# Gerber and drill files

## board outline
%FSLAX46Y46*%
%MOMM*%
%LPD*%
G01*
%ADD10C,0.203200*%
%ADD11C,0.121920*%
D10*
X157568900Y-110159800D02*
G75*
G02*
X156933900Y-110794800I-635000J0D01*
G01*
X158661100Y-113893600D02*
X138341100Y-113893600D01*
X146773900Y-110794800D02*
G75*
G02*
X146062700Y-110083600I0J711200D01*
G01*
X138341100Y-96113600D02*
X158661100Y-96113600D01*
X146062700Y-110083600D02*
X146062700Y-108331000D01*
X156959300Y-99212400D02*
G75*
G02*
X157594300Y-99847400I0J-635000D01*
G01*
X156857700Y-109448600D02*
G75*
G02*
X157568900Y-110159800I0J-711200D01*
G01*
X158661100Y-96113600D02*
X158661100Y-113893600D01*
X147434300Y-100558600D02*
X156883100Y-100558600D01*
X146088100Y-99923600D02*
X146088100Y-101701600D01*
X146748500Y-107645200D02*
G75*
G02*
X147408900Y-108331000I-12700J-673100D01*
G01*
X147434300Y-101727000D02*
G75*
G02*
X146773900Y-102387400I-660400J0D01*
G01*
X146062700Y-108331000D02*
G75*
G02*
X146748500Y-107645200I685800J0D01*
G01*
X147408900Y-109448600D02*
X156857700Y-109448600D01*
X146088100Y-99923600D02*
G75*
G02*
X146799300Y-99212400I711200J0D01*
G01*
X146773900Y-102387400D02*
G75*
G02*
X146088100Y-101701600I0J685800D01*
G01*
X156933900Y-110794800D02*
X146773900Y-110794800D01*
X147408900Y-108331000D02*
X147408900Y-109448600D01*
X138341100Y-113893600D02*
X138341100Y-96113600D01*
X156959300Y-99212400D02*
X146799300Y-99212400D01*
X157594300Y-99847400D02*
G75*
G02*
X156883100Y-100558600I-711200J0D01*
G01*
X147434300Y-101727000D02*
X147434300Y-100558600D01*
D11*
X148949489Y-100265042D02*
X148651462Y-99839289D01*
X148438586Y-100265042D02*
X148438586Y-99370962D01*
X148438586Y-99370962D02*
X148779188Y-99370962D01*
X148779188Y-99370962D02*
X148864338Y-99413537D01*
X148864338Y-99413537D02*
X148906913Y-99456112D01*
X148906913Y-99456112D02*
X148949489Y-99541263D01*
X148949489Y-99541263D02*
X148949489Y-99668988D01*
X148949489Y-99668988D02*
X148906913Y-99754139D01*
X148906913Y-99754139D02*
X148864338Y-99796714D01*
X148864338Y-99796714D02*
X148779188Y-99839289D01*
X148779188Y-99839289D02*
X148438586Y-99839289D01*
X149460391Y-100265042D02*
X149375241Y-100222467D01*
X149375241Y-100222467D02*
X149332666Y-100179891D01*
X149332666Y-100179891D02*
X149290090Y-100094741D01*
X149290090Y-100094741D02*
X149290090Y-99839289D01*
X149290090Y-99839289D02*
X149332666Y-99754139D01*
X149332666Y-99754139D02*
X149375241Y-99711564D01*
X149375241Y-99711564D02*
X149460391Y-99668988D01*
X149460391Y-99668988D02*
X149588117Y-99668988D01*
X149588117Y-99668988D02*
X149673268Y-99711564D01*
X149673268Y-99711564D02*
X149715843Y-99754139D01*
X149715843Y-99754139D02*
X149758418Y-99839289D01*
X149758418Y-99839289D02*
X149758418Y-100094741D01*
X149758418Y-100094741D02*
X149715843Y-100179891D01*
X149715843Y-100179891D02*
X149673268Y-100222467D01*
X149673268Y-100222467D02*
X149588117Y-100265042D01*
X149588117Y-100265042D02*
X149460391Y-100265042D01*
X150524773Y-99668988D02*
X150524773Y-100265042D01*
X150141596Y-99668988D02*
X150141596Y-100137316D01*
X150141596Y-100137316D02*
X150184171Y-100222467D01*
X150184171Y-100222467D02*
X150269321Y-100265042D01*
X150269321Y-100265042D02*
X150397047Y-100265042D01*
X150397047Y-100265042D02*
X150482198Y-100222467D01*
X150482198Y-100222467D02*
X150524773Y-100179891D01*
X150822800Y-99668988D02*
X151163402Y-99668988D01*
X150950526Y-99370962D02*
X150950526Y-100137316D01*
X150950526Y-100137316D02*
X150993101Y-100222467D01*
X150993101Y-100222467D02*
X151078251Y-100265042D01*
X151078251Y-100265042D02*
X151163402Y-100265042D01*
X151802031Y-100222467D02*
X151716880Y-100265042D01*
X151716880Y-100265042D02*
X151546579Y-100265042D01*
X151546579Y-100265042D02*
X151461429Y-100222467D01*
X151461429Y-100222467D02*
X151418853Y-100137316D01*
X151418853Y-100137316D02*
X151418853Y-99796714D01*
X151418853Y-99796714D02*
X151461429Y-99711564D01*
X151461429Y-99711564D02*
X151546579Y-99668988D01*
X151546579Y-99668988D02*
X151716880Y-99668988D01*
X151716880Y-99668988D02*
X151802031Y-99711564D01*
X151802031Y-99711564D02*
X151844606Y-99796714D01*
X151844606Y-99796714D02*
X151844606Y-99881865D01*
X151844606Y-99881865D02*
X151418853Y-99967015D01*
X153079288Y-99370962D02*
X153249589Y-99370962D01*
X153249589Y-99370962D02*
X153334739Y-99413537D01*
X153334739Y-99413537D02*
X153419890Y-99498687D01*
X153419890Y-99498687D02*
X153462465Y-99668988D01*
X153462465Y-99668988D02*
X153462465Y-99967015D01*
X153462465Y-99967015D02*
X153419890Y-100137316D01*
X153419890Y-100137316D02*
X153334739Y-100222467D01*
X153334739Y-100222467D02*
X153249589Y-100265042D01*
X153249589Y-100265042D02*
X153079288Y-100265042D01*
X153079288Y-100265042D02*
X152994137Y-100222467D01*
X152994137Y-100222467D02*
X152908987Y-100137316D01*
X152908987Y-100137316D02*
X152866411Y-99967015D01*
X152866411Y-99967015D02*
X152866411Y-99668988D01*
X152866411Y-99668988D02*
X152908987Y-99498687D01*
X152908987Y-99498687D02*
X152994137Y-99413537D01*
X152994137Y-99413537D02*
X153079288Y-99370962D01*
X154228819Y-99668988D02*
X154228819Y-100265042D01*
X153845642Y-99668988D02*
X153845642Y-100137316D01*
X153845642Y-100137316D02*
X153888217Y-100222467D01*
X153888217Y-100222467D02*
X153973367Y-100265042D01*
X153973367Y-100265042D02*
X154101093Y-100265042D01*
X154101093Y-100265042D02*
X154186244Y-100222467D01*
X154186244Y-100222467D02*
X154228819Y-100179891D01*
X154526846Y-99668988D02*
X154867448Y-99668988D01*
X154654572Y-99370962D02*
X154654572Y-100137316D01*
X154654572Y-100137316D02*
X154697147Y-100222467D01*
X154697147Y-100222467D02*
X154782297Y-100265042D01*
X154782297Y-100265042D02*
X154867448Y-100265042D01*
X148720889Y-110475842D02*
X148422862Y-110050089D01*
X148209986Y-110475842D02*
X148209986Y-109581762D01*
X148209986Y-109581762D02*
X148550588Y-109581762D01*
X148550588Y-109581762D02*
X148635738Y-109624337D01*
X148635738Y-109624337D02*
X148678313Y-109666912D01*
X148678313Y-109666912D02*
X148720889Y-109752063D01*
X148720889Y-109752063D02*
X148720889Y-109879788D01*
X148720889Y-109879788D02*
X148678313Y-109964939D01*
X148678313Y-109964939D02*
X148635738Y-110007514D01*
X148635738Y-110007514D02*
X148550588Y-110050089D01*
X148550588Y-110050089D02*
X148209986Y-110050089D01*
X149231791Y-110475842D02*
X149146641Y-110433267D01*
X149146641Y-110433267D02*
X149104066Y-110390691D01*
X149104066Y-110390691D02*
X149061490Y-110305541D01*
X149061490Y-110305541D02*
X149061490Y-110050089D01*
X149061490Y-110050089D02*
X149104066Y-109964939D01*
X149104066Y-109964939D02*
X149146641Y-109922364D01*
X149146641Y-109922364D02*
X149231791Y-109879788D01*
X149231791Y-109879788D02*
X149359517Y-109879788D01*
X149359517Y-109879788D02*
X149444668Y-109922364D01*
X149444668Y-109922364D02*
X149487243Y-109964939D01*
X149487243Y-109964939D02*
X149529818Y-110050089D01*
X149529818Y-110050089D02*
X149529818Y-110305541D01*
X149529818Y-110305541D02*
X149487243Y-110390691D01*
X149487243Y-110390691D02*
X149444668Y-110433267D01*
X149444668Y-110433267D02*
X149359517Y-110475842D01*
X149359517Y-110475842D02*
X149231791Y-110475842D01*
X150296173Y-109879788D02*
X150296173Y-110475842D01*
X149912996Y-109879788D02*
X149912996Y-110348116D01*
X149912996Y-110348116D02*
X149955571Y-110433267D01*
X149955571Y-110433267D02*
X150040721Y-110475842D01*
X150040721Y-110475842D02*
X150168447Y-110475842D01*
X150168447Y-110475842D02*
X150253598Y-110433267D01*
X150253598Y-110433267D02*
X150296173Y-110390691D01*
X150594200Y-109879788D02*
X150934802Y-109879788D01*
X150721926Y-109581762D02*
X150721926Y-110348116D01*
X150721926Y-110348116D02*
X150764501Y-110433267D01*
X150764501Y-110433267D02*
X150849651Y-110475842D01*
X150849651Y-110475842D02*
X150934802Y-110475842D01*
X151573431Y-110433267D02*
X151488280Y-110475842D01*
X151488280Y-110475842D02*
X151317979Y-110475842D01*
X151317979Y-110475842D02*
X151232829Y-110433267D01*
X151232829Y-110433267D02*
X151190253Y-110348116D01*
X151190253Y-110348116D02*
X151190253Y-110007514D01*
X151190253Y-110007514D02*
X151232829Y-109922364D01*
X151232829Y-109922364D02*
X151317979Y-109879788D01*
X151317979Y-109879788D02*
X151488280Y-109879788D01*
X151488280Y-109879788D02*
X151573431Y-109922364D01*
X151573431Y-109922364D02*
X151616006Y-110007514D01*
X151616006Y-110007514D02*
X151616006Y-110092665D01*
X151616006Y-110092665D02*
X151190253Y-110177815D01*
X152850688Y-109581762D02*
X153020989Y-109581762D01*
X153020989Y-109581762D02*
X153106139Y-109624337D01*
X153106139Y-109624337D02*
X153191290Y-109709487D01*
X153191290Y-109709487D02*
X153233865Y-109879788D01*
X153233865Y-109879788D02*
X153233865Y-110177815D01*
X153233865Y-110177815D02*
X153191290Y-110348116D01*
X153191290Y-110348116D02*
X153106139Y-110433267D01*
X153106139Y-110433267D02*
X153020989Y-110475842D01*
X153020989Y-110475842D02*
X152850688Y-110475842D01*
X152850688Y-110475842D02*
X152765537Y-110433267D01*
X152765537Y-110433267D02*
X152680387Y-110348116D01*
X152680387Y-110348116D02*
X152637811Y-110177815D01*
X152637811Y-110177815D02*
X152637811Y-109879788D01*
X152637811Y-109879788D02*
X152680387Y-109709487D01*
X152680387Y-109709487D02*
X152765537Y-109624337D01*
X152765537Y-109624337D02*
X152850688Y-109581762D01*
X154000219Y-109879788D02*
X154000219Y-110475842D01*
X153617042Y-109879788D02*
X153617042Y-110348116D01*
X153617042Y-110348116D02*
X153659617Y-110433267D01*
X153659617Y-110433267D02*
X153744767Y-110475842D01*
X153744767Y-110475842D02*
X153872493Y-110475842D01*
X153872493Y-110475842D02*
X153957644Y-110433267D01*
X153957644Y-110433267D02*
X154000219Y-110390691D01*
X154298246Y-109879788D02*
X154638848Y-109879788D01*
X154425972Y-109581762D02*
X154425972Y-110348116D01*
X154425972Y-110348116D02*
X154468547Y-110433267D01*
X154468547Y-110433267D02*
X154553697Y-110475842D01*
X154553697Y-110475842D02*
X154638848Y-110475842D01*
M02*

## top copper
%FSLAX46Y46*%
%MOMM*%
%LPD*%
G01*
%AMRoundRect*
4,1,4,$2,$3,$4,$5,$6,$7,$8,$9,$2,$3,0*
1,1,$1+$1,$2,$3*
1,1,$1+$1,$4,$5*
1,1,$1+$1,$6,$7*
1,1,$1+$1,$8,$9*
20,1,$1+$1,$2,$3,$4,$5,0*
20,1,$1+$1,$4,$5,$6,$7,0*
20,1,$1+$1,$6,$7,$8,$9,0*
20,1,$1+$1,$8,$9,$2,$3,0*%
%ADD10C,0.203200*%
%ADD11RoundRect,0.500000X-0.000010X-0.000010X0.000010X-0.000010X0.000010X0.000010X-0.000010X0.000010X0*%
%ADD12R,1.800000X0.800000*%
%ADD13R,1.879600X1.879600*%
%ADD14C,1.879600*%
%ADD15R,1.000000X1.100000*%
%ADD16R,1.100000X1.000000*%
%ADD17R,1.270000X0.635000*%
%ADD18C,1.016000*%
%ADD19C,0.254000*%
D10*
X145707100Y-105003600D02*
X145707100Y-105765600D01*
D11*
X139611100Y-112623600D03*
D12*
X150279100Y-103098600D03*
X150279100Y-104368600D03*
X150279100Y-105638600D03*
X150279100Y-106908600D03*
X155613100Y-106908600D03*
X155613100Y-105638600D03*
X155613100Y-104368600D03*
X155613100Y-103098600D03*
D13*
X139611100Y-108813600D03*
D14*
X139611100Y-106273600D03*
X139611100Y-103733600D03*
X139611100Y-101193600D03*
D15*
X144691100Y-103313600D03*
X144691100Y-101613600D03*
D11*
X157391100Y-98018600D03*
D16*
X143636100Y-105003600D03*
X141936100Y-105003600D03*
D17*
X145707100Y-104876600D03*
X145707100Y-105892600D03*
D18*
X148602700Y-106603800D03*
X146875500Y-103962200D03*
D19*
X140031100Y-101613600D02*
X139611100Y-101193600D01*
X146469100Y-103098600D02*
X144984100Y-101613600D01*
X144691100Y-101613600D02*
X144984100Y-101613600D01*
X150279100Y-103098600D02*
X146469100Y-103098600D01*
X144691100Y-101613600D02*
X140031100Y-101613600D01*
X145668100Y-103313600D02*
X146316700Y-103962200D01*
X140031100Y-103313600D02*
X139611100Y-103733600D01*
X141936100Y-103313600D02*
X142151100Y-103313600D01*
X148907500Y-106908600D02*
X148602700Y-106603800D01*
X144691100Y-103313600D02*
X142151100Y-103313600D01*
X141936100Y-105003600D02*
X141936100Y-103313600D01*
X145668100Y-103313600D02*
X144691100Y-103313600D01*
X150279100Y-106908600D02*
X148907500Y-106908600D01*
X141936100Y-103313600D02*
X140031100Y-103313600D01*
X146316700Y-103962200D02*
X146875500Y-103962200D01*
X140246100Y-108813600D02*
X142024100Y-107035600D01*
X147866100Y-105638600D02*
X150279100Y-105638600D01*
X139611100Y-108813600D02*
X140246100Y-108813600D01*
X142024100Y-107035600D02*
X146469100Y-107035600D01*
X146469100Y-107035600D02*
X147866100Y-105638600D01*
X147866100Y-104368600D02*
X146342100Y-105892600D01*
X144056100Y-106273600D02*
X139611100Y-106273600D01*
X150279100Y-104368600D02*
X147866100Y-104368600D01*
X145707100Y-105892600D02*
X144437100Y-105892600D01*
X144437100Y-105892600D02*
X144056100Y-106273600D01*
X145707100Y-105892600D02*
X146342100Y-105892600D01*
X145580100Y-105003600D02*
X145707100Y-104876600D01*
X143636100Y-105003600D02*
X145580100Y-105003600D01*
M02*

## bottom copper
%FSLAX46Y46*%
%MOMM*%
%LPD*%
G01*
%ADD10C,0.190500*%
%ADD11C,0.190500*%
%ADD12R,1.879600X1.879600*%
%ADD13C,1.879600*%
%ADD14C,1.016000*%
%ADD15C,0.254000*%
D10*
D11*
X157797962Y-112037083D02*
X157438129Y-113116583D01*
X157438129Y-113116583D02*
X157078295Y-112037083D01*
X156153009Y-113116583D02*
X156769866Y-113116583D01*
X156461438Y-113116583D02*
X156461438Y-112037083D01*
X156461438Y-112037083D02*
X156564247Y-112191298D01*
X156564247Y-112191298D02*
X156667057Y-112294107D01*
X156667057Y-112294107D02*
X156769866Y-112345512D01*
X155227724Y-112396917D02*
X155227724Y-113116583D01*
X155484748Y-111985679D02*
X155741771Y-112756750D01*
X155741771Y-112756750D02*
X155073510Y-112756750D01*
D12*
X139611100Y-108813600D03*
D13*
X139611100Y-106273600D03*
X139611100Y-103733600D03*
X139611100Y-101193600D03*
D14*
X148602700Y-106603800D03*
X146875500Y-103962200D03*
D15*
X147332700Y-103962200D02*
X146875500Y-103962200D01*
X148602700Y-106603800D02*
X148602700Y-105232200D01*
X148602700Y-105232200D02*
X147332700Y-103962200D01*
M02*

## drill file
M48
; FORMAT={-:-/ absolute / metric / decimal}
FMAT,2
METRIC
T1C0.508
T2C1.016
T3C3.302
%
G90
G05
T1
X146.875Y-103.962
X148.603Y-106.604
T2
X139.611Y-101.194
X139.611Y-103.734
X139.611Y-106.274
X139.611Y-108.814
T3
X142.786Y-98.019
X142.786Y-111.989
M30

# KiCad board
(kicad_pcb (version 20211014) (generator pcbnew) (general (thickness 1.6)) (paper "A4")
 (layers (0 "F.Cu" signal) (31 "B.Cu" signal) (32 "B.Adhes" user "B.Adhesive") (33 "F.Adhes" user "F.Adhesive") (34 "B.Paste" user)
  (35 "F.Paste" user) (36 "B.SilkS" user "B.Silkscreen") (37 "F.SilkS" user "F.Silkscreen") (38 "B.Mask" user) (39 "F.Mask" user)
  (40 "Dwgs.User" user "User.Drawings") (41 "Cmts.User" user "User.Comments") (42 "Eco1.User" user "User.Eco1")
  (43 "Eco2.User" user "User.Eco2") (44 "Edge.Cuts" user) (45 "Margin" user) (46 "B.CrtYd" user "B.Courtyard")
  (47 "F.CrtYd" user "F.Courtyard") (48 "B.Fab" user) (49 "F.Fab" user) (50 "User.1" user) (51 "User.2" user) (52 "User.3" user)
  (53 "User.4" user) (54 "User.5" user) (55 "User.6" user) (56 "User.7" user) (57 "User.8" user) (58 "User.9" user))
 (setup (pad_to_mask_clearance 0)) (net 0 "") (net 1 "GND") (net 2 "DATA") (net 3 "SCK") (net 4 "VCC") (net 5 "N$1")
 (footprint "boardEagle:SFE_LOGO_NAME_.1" (layer "F.Cu") (at 145.2245 99.568)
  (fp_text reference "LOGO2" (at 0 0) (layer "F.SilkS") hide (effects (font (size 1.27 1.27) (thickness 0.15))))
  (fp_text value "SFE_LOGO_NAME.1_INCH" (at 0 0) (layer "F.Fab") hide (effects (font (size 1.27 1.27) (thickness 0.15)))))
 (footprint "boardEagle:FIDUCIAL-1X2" (layer "F.Cu") (at 139.6111 112.6236)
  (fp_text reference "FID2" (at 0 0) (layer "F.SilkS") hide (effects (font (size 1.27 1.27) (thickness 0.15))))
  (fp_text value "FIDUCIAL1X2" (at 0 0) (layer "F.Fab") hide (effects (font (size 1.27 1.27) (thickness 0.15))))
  (pad "1" smd roundrect (at 0 0) (size 1 1) (layers "F.Cu" "F.Mask") (roundrect_rratio 0.5) (solder_mask_margin 0.1016)))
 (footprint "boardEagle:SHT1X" (layer "F.Cu") (at 152.9461 105.0036)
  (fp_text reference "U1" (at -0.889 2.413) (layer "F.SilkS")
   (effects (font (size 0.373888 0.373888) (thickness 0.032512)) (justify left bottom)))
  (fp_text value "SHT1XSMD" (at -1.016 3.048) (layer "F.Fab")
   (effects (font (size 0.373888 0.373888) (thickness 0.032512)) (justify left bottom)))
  (pad "1" smd rect (at -2.667 -1.905 180) (size 1.8 0.8) (layers "F.Cu" "F.Paste" "F.Mask") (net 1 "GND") (solder_mask_margin 0.1016))
  (pad "2" smd rect (at -2.667 -0.635 180) (size 1.8 0.8) (layers "F.Cu" "F.Paste" "F.Mask") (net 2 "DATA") (solder_mask_margin 0.1016))
  (pad "3" smd rect (at -2.667 0.635 180) (size 1.8 0.8) (layers "F.Cu" "F.Paste" "F.Mask") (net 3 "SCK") (solder_mask_margin 0.1016))
  (pad "4" smd rect (at -2.667 1.905 180) (size 1.8 0.8) (layers "F.Cu" "F.Paste" "F.Mask") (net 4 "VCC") (solder_mask_margin 0.1016))
  (pad "5" smd rect (at 2.667 1.905 180) (size 1.8 0.8) (layers "F.Cu" "F.Paste" "F.Mask") (solder_mask_margin 0.1016))
  (pad "6" smd rect (at 2.667 0.635 180) (size 1.8 0.8) (layers "F.Cu" "F.Paste" "F.Mask") (solder_mask_margin 0.1016))
  (pad "7" smd rect (at 2.667 -0.635 180) (size 1.8 0.8) (layers "F.Cu" "F.Paste" "F.Mask") (solder_mask_margin 0.1016))
  (pad "8" smd rect (at 2.667 -1.905 180) (size 1.8 0.8) (layers "F.Cu" "F.Paste" "F.Mask") (solder_mask_margin 0.1016)))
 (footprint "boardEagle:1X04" (layer "F.Cu") (at 139.6111 108.8136 90)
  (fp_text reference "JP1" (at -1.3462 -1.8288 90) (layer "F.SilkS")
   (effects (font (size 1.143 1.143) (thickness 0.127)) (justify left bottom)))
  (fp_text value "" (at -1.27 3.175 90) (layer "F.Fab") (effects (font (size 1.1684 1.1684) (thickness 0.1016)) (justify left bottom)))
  (pad "1" thru_hole rect (at 0 0 180) (size 1.8796 1.8796) (drill 1.016) (layers *.Cu *.Mask) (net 3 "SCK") (solder_mask_margin 0.1016))
  (pad "2" thru_hole circle (at 2.54 0 180) (size 1.8796 1.8796) (drill 1.016) (layers *.Cu *.Mask) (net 2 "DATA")
   (solder_mask_margin 0.1016))
  (pad "3" thru_hole circle (at 5.08 0 180) (size 1.8796 1.8796) (drill 1.016) (layers *.Cu *.Mask) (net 4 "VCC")
   (solder_mask_margin 0.1016))
  (pad "4" thru_hole circle (at 7.62 0 180) (size 1.8796 1.8796) (drill 1.016) (layers *.Cu *.Mask) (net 1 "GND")
   (solder_mask_margin 0.1016)))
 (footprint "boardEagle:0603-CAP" (layer "F.Cu") (at 144.6911 102.4636 90)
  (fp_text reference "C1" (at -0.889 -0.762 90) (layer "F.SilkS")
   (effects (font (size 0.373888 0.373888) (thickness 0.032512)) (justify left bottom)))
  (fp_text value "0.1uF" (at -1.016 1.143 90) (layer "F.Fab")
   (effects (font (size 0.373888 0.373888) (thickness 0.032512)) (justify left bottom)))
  (pad "1" smd rect (at -0.85 0 90) (size 1.1 1) (layers "F.Cu" "F.Paste" "F.Mask") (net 4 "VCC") (solder_mask_margin 0.1016))
  (pad "2" smd rect (at 0.85 0 90) (size 1.1 1) (layers "F.Cu" "F.Paste" "F.Mask") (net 1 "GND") (solder_mask_margin 0.1016)))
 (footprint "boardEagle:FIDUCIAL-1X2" (layer "F.Cu") (at 157.3911 98.0186)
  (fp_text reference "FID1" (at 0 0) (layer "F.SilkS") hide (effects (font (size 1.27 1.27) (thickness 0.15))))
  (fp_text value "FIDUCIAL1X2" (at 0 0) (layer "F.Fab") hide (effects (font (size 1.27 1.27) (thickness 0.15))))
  (pad "1" smd roundrect (at 0 0) (size 1 1) (layers "F.Cu" "F.Mask") (roundrect_rratio 0.5) (solder_mask_margin 0.1016)))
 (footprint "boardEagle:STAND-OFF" (layer "F.Cu") (at 142.7861 111.9886)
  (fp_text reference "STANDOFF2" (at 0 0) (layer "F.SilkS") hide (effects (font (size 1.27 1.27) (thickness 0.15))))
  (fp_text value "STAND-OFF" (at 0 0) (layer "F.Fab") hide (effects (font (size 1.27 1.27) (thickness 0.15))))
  (pad "" np_thru_hole circle (at 0 0) (size 3.302 3.302) (drill 3.302) (layers *.Cu *.Mask)))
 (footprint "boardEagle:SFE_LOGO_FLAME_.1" (layer "F.Cu") (at 138.5189 99.695)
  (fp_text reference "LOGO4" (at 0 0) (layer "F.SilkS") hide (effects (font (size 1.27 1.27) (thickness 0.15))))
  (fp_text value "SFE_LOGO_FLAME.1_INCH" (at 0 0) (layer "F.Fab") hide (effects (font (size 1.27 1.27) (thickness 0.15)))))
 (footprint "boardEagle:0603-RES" (layer "F.Cu") (at 142.7861 105.0036 180)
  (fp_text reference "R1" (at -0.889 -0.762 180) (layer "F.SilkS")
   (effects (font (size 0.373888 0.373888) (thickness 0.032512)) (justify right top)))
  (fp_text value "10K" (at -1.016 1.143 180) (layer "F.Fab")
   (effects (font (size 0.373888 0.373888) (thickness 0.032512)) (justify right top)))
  (pad "1" smd rect (at -0.85 0 180) (size 1.1 1) (layers "F.Cu" "F.Paste" "F.Mask") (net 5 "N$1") (solder_mask_margin 0.1016))
  (pad "2" smd rect (at 0.85 0 180) (size 1.1 1) (layers "F.Cu" "F.Paste" "F.Mask") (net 4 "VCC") (solder_mask_margin 0.1016)))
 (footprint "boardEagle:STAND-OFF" (layer "F.Cu") (at 142.7861 98.0186)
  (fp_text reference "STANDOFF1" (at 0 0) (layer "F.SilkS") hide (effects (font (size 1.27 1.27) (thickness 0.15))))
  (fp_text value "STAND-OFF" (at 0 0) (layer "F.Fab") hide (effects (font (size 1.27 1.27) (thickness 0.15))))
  (pad "" np_thru_hole circle (at 0 0) (size 3.302 3.302) (drill 3.302) (layers *.Cu *.Mask)))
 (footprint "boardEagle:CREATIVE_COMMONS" (layer "F.Cu") (at 120.5611 124.0536)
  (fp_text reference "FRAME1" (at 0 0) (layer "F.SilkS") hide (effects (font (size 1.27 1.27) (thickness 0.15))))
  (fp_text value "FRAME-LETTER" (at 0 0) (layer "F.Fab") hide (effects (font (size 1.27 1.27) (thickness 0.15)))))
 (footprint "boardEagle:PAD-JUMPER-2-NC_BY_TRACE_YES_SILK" (layer "F.Cu") (at 145.7071 105.3846 -90)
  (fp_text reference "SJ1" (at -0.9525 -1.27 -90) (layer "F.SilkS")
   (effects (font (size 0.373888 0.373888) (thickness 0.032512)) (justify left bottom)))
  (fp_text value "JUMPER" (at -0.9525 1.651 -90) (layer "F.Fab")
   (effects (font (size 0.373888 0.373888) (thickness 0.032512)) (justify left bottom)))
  (fp_line (start -0.381 0) (end 0.381 0) (layer "F.Cu") (width 0.2032))
  (pad "1" smd rect (at -0.508 0 270) (size 0.635 1.27) (layers "F.Cu" "F.Mask") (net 5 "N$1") (solder_mask_margin 0.1016))
  (pad "2" smd rect (at 0.508 0 270) (size 0.635 1.27) (layers "F.Cu" "F.Mask") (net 2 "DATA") (solder_mask_margin 0.1016)))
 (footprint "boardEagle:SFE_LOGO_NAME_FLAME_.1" (layer "B.Cu") (at 158.7373 106.5276 180)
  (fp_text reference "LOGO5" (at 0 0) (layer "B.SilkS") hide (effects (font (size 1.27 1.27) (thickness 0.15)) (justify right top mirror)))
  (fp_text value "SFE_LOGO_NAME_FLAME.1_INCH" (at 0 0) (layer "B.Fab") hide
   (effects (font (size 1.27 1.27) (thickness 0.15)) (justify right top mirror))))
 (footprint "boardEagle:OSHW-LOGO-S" (layer "B.Cu") (at 152.3111 112.4966 180)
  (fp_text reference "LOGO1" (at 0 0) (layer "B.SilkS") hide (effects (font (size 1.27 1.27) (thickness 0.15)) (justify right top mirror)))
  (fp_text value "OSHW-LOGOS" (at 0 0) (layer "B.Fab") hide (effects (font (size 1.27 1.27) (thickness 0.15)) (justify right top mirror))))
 (gr_arc (start 157.5689 110.1598) (mid 157.382913 110.608813) (end 156.9339 110.7948) (layer "Edge.Cuts") (width 0.2032))
 (gr_line (start 158.6611 113.8936) (end 138.3411 113.8936) (layer "Edge.Cuts") (width 0.2032))
 (gr_arc (start 146.7739 110.7948) (mid 146.271006 110.586494) (end 146.0627 110.0836) (layer "Edge.Cuts") (width 0.2032))
 (gr_line (start 138.3411 96.1136) (end 158.6611 96.1136) (layer "Edge.Cuts") (width 0.2032))
 (gr_line (start 146.0627 110.0836) (end 146.0627 108.331) (layer "Edge.Cuts") (width 0.2032))
 (gr_arc (start 156.9593 99.2124) (mid 157.408313 99.398387) (end 157.5943 99.8474) (layer "Edge.Cuts") (width 0.2032))
 (gr_arc (start 156.8577 109.4486) (mid 157.360594 109.656906) (end 157.5689 110.1598) (layer "Edge.Cuts") (width 0.2032))
 (gr_line (start 158.6611 96.1136) (end 158.6611 113.8936) (layer "Edge.Cuts") (width 0.2032))
 (gr_line (start 147.4343 100.5586) (end 156.8831 100.5586) (layer "Edge.Cuts") (width 0.2032))
 (gr_line (start 146.0881 99.9236) (end 146.0881 101.7016) (layer "Edge.Cuts") (width 0.2032))
 (gr_arc (start 146.7485 107.6452) (mid 147.220734 107.851327) (end 147.4089 108.331) (layer "Edge.Cuts") (width 0.2032))
 (gr_arc (start 147.4343 101.727) (mid 147.240873 102.193973) (end 146.7739 102.3874) (layer "Edge.Cuts") (width 0.2032))
 (gr_arc (start 146.0627 108.331) (mid 146.263566 107.846066) (end 146.7485 107.6452) (layer "Edge.Cuts") (width 0.2032))
 (gr_line (start 147.4089 109.4486) (end 156.8577 109.4486) (layer "Edge.Cuts") (width 0.2032))
 (gr_arc (start 146.0881 99.9236) (mid 146.296406 99.420706) (end 146.7993 99.2124) (layer "Edge.Cuts") (width 0.2032))
 (gr_arc (start 146.7739 102.3874) (mid 146.288966 102.186534) (end 146.0881 101.7016) (layer "Edge.Cuts") (width 0.2032))
 (gr_line (start 156.9339 110.7948) (end 146.7739 110.7948) (layer "Edge.Cuts") (width 0.2032))
 (gr_line (start 147.4089 108.331) (end 147.4089 109.4486) (layer "Edge.Cuts") (width 0.2032))
 (gr_line (start 138.3411 113.8936) (end 138.3411 96.1136) (layer "Edge.Cuts") (width 0.2032))
 (gr_line (start 156.9593 99.2124) (end 146.7993 99.2124) (layer "Edge.Cuts") (width 0.2032))
 (gr_arc (start 157.5943 99.8474) (mid 157.385994 100.350294) (end 156.8831 100.5586) (layer "Edge.Cuts") (width 0.2032))
 (gr_line (start 147.4343 101.727) (end 147.4343 100.5586) (layer "Edge.Cuts") (width 0.2032))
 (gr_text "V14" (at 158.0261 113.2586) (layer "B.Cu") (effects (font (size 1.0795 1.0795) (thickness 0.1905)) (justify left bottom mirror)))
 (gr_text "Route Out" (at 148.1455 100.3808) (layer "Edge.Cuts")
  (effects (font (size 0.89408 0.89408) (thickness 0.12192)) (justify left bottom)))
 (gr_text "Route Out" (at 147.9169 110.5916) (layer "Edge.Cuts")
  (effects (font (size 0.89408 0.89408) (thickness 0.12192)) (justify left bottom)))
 (segment (start 140.0311 101.6136) (end 139.6111 101.1936) (width 0.254) (layer "F.Cu") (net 1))
 (segment (start 146.4691 103.0986) (end 144.9841 101.6136) (width 0.254) (layer "F.Cu") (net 1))
 (segment (start 144.6911 101.6136) (end 144.9841 101.6136) (width 0.254) (layer "F.Cu") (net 1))
 (segment (start 150.2791 103.0986) (end 146.4691 103.0986) (width 0.254) (layer "F.Cu") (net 1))
 (segment (start 144.6911 101.6136) (end 140.0311 101.6136) (width 0.254) (layer "F.Cu") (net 1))
 (segment (start 145.6681 103.3136) (end 146.3167 103.9622) (width 0.254) (layer "F.Cu") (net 4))
 (segment (start 140.0311 103.3136) (end 139.6111 103.7336) (width 0.254) (layer "F.Cu") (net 4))
 (segment (start 141.9361 103.3136) (end 142.1511 103.3136) (width 0.254) (layer "F.Cu") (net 4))
 (segment (start 148.9075 106.9086) (end 148.6027 106.6038) (width 0.254) (layer "F.Cu") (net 4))
 (segment (start 144.6911 103.3136) (end 142.1511 103.3136) (width 0.254) (layer "F.Cu") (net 4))
 (segment (start 141.9361 105.0036) (end 141.9361 103.3136) (width 0.254) (layer "F.Cu") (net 4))
 (segment (start 145.6681 103.3136) (end 144.6911 103.3136) (width 0.254) (layer "F.Cu") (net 4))
 (segment (start 150.2791 106.9086) (end 148.9075 106.9086) (width 0.254) (layer "F.Cu") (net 4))
 (segment (start 141.9361 103.3136) (end 140.0311 103.3136) (width 0.254) (layer "F.Cu") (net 4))
 (segment (start 146.3167 103.9622) (end 146.8755 103.9622) (width 0.254) (layer "F.Cu") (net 4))
 (via (at 148.6027 106.6038) (size 1.016) (drill 0.508) (layers "F.Cu" "B.Cu") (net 4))
 (via (at 146.8755 103.9622) (size 1.016) (drill 0.508) (layers "F.Cu" "B.Cu") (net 4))
 (segment (start 147.3327 103.9622) (end 146.8755 103.9622) (width 0.254) (layer "B.Cu") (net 4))
 (segment (start 148.6027 106.6038) (end 148.6027 105.2322) (width 0.254) (layer "B.Cu") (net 4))
 (segment (start 148.6027 105.2322) (end 147.3327 103.9622) (width 0.254) (layer "B.Cu") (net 4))
 (segment (start 140.2461 108.8136) (end 142.0241 107.0356) (width 0.254) (layer "F.Cu") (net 3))
 (segment (start 147.8661 105.6386) (end 150.2791 105.6386) (width 0.254) (layer "F.Cu") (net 3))
 (segment (start 139.6111 108.8136) (end 140.2461 108.8136) (width 0.254) (layer "F.Cu") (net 3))
 (segment (start 142.0241 107.0356) (end 146.4691 107.0356) (width 0.254) (layer "F.Cu") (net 3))
 (segment (start 146.4691 107.0356) (end 147.8661 105.6386) (width 0.254) (layer "F.Cu") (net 3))
 (segment (start 147.8661 104.3686) (end 146.3421 105.8926) (width 0.254) (layer "F.Cu") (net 2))
 (segment (start 144.0561 106.2736) (end 139.6111 106.2736) (width 0.254) (layer "F.Cu") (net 2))
 (segment (start 150.2791 104.3686) (end 147.8661 104.3686) (width 0.254) (layer "F.Cu") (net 2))
 (segment (start 145.7071 105.8926) (end 144.4371 105.8926) (width 0.254) (layer "F.Cu") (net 2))
 (segment (start 144.4371 105.8926) (end 144.0561 106.2736) (width 0.254) (layer "F.Cu") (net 2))
 (segment (start 145.7071 105.8926) (end 146.3421 105.8926) (width 0.254) (layer "F.Cu") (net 2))
 (segment (start 145.5801 105.0036) (end 145.7071 104.8766) (width 0.254) (layer "F.Cu") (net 5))
 (segment (start 143.6361 105.0036) (end 145.5801 105.0036) (width 0.254) (layer "F.Cu") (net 5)))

